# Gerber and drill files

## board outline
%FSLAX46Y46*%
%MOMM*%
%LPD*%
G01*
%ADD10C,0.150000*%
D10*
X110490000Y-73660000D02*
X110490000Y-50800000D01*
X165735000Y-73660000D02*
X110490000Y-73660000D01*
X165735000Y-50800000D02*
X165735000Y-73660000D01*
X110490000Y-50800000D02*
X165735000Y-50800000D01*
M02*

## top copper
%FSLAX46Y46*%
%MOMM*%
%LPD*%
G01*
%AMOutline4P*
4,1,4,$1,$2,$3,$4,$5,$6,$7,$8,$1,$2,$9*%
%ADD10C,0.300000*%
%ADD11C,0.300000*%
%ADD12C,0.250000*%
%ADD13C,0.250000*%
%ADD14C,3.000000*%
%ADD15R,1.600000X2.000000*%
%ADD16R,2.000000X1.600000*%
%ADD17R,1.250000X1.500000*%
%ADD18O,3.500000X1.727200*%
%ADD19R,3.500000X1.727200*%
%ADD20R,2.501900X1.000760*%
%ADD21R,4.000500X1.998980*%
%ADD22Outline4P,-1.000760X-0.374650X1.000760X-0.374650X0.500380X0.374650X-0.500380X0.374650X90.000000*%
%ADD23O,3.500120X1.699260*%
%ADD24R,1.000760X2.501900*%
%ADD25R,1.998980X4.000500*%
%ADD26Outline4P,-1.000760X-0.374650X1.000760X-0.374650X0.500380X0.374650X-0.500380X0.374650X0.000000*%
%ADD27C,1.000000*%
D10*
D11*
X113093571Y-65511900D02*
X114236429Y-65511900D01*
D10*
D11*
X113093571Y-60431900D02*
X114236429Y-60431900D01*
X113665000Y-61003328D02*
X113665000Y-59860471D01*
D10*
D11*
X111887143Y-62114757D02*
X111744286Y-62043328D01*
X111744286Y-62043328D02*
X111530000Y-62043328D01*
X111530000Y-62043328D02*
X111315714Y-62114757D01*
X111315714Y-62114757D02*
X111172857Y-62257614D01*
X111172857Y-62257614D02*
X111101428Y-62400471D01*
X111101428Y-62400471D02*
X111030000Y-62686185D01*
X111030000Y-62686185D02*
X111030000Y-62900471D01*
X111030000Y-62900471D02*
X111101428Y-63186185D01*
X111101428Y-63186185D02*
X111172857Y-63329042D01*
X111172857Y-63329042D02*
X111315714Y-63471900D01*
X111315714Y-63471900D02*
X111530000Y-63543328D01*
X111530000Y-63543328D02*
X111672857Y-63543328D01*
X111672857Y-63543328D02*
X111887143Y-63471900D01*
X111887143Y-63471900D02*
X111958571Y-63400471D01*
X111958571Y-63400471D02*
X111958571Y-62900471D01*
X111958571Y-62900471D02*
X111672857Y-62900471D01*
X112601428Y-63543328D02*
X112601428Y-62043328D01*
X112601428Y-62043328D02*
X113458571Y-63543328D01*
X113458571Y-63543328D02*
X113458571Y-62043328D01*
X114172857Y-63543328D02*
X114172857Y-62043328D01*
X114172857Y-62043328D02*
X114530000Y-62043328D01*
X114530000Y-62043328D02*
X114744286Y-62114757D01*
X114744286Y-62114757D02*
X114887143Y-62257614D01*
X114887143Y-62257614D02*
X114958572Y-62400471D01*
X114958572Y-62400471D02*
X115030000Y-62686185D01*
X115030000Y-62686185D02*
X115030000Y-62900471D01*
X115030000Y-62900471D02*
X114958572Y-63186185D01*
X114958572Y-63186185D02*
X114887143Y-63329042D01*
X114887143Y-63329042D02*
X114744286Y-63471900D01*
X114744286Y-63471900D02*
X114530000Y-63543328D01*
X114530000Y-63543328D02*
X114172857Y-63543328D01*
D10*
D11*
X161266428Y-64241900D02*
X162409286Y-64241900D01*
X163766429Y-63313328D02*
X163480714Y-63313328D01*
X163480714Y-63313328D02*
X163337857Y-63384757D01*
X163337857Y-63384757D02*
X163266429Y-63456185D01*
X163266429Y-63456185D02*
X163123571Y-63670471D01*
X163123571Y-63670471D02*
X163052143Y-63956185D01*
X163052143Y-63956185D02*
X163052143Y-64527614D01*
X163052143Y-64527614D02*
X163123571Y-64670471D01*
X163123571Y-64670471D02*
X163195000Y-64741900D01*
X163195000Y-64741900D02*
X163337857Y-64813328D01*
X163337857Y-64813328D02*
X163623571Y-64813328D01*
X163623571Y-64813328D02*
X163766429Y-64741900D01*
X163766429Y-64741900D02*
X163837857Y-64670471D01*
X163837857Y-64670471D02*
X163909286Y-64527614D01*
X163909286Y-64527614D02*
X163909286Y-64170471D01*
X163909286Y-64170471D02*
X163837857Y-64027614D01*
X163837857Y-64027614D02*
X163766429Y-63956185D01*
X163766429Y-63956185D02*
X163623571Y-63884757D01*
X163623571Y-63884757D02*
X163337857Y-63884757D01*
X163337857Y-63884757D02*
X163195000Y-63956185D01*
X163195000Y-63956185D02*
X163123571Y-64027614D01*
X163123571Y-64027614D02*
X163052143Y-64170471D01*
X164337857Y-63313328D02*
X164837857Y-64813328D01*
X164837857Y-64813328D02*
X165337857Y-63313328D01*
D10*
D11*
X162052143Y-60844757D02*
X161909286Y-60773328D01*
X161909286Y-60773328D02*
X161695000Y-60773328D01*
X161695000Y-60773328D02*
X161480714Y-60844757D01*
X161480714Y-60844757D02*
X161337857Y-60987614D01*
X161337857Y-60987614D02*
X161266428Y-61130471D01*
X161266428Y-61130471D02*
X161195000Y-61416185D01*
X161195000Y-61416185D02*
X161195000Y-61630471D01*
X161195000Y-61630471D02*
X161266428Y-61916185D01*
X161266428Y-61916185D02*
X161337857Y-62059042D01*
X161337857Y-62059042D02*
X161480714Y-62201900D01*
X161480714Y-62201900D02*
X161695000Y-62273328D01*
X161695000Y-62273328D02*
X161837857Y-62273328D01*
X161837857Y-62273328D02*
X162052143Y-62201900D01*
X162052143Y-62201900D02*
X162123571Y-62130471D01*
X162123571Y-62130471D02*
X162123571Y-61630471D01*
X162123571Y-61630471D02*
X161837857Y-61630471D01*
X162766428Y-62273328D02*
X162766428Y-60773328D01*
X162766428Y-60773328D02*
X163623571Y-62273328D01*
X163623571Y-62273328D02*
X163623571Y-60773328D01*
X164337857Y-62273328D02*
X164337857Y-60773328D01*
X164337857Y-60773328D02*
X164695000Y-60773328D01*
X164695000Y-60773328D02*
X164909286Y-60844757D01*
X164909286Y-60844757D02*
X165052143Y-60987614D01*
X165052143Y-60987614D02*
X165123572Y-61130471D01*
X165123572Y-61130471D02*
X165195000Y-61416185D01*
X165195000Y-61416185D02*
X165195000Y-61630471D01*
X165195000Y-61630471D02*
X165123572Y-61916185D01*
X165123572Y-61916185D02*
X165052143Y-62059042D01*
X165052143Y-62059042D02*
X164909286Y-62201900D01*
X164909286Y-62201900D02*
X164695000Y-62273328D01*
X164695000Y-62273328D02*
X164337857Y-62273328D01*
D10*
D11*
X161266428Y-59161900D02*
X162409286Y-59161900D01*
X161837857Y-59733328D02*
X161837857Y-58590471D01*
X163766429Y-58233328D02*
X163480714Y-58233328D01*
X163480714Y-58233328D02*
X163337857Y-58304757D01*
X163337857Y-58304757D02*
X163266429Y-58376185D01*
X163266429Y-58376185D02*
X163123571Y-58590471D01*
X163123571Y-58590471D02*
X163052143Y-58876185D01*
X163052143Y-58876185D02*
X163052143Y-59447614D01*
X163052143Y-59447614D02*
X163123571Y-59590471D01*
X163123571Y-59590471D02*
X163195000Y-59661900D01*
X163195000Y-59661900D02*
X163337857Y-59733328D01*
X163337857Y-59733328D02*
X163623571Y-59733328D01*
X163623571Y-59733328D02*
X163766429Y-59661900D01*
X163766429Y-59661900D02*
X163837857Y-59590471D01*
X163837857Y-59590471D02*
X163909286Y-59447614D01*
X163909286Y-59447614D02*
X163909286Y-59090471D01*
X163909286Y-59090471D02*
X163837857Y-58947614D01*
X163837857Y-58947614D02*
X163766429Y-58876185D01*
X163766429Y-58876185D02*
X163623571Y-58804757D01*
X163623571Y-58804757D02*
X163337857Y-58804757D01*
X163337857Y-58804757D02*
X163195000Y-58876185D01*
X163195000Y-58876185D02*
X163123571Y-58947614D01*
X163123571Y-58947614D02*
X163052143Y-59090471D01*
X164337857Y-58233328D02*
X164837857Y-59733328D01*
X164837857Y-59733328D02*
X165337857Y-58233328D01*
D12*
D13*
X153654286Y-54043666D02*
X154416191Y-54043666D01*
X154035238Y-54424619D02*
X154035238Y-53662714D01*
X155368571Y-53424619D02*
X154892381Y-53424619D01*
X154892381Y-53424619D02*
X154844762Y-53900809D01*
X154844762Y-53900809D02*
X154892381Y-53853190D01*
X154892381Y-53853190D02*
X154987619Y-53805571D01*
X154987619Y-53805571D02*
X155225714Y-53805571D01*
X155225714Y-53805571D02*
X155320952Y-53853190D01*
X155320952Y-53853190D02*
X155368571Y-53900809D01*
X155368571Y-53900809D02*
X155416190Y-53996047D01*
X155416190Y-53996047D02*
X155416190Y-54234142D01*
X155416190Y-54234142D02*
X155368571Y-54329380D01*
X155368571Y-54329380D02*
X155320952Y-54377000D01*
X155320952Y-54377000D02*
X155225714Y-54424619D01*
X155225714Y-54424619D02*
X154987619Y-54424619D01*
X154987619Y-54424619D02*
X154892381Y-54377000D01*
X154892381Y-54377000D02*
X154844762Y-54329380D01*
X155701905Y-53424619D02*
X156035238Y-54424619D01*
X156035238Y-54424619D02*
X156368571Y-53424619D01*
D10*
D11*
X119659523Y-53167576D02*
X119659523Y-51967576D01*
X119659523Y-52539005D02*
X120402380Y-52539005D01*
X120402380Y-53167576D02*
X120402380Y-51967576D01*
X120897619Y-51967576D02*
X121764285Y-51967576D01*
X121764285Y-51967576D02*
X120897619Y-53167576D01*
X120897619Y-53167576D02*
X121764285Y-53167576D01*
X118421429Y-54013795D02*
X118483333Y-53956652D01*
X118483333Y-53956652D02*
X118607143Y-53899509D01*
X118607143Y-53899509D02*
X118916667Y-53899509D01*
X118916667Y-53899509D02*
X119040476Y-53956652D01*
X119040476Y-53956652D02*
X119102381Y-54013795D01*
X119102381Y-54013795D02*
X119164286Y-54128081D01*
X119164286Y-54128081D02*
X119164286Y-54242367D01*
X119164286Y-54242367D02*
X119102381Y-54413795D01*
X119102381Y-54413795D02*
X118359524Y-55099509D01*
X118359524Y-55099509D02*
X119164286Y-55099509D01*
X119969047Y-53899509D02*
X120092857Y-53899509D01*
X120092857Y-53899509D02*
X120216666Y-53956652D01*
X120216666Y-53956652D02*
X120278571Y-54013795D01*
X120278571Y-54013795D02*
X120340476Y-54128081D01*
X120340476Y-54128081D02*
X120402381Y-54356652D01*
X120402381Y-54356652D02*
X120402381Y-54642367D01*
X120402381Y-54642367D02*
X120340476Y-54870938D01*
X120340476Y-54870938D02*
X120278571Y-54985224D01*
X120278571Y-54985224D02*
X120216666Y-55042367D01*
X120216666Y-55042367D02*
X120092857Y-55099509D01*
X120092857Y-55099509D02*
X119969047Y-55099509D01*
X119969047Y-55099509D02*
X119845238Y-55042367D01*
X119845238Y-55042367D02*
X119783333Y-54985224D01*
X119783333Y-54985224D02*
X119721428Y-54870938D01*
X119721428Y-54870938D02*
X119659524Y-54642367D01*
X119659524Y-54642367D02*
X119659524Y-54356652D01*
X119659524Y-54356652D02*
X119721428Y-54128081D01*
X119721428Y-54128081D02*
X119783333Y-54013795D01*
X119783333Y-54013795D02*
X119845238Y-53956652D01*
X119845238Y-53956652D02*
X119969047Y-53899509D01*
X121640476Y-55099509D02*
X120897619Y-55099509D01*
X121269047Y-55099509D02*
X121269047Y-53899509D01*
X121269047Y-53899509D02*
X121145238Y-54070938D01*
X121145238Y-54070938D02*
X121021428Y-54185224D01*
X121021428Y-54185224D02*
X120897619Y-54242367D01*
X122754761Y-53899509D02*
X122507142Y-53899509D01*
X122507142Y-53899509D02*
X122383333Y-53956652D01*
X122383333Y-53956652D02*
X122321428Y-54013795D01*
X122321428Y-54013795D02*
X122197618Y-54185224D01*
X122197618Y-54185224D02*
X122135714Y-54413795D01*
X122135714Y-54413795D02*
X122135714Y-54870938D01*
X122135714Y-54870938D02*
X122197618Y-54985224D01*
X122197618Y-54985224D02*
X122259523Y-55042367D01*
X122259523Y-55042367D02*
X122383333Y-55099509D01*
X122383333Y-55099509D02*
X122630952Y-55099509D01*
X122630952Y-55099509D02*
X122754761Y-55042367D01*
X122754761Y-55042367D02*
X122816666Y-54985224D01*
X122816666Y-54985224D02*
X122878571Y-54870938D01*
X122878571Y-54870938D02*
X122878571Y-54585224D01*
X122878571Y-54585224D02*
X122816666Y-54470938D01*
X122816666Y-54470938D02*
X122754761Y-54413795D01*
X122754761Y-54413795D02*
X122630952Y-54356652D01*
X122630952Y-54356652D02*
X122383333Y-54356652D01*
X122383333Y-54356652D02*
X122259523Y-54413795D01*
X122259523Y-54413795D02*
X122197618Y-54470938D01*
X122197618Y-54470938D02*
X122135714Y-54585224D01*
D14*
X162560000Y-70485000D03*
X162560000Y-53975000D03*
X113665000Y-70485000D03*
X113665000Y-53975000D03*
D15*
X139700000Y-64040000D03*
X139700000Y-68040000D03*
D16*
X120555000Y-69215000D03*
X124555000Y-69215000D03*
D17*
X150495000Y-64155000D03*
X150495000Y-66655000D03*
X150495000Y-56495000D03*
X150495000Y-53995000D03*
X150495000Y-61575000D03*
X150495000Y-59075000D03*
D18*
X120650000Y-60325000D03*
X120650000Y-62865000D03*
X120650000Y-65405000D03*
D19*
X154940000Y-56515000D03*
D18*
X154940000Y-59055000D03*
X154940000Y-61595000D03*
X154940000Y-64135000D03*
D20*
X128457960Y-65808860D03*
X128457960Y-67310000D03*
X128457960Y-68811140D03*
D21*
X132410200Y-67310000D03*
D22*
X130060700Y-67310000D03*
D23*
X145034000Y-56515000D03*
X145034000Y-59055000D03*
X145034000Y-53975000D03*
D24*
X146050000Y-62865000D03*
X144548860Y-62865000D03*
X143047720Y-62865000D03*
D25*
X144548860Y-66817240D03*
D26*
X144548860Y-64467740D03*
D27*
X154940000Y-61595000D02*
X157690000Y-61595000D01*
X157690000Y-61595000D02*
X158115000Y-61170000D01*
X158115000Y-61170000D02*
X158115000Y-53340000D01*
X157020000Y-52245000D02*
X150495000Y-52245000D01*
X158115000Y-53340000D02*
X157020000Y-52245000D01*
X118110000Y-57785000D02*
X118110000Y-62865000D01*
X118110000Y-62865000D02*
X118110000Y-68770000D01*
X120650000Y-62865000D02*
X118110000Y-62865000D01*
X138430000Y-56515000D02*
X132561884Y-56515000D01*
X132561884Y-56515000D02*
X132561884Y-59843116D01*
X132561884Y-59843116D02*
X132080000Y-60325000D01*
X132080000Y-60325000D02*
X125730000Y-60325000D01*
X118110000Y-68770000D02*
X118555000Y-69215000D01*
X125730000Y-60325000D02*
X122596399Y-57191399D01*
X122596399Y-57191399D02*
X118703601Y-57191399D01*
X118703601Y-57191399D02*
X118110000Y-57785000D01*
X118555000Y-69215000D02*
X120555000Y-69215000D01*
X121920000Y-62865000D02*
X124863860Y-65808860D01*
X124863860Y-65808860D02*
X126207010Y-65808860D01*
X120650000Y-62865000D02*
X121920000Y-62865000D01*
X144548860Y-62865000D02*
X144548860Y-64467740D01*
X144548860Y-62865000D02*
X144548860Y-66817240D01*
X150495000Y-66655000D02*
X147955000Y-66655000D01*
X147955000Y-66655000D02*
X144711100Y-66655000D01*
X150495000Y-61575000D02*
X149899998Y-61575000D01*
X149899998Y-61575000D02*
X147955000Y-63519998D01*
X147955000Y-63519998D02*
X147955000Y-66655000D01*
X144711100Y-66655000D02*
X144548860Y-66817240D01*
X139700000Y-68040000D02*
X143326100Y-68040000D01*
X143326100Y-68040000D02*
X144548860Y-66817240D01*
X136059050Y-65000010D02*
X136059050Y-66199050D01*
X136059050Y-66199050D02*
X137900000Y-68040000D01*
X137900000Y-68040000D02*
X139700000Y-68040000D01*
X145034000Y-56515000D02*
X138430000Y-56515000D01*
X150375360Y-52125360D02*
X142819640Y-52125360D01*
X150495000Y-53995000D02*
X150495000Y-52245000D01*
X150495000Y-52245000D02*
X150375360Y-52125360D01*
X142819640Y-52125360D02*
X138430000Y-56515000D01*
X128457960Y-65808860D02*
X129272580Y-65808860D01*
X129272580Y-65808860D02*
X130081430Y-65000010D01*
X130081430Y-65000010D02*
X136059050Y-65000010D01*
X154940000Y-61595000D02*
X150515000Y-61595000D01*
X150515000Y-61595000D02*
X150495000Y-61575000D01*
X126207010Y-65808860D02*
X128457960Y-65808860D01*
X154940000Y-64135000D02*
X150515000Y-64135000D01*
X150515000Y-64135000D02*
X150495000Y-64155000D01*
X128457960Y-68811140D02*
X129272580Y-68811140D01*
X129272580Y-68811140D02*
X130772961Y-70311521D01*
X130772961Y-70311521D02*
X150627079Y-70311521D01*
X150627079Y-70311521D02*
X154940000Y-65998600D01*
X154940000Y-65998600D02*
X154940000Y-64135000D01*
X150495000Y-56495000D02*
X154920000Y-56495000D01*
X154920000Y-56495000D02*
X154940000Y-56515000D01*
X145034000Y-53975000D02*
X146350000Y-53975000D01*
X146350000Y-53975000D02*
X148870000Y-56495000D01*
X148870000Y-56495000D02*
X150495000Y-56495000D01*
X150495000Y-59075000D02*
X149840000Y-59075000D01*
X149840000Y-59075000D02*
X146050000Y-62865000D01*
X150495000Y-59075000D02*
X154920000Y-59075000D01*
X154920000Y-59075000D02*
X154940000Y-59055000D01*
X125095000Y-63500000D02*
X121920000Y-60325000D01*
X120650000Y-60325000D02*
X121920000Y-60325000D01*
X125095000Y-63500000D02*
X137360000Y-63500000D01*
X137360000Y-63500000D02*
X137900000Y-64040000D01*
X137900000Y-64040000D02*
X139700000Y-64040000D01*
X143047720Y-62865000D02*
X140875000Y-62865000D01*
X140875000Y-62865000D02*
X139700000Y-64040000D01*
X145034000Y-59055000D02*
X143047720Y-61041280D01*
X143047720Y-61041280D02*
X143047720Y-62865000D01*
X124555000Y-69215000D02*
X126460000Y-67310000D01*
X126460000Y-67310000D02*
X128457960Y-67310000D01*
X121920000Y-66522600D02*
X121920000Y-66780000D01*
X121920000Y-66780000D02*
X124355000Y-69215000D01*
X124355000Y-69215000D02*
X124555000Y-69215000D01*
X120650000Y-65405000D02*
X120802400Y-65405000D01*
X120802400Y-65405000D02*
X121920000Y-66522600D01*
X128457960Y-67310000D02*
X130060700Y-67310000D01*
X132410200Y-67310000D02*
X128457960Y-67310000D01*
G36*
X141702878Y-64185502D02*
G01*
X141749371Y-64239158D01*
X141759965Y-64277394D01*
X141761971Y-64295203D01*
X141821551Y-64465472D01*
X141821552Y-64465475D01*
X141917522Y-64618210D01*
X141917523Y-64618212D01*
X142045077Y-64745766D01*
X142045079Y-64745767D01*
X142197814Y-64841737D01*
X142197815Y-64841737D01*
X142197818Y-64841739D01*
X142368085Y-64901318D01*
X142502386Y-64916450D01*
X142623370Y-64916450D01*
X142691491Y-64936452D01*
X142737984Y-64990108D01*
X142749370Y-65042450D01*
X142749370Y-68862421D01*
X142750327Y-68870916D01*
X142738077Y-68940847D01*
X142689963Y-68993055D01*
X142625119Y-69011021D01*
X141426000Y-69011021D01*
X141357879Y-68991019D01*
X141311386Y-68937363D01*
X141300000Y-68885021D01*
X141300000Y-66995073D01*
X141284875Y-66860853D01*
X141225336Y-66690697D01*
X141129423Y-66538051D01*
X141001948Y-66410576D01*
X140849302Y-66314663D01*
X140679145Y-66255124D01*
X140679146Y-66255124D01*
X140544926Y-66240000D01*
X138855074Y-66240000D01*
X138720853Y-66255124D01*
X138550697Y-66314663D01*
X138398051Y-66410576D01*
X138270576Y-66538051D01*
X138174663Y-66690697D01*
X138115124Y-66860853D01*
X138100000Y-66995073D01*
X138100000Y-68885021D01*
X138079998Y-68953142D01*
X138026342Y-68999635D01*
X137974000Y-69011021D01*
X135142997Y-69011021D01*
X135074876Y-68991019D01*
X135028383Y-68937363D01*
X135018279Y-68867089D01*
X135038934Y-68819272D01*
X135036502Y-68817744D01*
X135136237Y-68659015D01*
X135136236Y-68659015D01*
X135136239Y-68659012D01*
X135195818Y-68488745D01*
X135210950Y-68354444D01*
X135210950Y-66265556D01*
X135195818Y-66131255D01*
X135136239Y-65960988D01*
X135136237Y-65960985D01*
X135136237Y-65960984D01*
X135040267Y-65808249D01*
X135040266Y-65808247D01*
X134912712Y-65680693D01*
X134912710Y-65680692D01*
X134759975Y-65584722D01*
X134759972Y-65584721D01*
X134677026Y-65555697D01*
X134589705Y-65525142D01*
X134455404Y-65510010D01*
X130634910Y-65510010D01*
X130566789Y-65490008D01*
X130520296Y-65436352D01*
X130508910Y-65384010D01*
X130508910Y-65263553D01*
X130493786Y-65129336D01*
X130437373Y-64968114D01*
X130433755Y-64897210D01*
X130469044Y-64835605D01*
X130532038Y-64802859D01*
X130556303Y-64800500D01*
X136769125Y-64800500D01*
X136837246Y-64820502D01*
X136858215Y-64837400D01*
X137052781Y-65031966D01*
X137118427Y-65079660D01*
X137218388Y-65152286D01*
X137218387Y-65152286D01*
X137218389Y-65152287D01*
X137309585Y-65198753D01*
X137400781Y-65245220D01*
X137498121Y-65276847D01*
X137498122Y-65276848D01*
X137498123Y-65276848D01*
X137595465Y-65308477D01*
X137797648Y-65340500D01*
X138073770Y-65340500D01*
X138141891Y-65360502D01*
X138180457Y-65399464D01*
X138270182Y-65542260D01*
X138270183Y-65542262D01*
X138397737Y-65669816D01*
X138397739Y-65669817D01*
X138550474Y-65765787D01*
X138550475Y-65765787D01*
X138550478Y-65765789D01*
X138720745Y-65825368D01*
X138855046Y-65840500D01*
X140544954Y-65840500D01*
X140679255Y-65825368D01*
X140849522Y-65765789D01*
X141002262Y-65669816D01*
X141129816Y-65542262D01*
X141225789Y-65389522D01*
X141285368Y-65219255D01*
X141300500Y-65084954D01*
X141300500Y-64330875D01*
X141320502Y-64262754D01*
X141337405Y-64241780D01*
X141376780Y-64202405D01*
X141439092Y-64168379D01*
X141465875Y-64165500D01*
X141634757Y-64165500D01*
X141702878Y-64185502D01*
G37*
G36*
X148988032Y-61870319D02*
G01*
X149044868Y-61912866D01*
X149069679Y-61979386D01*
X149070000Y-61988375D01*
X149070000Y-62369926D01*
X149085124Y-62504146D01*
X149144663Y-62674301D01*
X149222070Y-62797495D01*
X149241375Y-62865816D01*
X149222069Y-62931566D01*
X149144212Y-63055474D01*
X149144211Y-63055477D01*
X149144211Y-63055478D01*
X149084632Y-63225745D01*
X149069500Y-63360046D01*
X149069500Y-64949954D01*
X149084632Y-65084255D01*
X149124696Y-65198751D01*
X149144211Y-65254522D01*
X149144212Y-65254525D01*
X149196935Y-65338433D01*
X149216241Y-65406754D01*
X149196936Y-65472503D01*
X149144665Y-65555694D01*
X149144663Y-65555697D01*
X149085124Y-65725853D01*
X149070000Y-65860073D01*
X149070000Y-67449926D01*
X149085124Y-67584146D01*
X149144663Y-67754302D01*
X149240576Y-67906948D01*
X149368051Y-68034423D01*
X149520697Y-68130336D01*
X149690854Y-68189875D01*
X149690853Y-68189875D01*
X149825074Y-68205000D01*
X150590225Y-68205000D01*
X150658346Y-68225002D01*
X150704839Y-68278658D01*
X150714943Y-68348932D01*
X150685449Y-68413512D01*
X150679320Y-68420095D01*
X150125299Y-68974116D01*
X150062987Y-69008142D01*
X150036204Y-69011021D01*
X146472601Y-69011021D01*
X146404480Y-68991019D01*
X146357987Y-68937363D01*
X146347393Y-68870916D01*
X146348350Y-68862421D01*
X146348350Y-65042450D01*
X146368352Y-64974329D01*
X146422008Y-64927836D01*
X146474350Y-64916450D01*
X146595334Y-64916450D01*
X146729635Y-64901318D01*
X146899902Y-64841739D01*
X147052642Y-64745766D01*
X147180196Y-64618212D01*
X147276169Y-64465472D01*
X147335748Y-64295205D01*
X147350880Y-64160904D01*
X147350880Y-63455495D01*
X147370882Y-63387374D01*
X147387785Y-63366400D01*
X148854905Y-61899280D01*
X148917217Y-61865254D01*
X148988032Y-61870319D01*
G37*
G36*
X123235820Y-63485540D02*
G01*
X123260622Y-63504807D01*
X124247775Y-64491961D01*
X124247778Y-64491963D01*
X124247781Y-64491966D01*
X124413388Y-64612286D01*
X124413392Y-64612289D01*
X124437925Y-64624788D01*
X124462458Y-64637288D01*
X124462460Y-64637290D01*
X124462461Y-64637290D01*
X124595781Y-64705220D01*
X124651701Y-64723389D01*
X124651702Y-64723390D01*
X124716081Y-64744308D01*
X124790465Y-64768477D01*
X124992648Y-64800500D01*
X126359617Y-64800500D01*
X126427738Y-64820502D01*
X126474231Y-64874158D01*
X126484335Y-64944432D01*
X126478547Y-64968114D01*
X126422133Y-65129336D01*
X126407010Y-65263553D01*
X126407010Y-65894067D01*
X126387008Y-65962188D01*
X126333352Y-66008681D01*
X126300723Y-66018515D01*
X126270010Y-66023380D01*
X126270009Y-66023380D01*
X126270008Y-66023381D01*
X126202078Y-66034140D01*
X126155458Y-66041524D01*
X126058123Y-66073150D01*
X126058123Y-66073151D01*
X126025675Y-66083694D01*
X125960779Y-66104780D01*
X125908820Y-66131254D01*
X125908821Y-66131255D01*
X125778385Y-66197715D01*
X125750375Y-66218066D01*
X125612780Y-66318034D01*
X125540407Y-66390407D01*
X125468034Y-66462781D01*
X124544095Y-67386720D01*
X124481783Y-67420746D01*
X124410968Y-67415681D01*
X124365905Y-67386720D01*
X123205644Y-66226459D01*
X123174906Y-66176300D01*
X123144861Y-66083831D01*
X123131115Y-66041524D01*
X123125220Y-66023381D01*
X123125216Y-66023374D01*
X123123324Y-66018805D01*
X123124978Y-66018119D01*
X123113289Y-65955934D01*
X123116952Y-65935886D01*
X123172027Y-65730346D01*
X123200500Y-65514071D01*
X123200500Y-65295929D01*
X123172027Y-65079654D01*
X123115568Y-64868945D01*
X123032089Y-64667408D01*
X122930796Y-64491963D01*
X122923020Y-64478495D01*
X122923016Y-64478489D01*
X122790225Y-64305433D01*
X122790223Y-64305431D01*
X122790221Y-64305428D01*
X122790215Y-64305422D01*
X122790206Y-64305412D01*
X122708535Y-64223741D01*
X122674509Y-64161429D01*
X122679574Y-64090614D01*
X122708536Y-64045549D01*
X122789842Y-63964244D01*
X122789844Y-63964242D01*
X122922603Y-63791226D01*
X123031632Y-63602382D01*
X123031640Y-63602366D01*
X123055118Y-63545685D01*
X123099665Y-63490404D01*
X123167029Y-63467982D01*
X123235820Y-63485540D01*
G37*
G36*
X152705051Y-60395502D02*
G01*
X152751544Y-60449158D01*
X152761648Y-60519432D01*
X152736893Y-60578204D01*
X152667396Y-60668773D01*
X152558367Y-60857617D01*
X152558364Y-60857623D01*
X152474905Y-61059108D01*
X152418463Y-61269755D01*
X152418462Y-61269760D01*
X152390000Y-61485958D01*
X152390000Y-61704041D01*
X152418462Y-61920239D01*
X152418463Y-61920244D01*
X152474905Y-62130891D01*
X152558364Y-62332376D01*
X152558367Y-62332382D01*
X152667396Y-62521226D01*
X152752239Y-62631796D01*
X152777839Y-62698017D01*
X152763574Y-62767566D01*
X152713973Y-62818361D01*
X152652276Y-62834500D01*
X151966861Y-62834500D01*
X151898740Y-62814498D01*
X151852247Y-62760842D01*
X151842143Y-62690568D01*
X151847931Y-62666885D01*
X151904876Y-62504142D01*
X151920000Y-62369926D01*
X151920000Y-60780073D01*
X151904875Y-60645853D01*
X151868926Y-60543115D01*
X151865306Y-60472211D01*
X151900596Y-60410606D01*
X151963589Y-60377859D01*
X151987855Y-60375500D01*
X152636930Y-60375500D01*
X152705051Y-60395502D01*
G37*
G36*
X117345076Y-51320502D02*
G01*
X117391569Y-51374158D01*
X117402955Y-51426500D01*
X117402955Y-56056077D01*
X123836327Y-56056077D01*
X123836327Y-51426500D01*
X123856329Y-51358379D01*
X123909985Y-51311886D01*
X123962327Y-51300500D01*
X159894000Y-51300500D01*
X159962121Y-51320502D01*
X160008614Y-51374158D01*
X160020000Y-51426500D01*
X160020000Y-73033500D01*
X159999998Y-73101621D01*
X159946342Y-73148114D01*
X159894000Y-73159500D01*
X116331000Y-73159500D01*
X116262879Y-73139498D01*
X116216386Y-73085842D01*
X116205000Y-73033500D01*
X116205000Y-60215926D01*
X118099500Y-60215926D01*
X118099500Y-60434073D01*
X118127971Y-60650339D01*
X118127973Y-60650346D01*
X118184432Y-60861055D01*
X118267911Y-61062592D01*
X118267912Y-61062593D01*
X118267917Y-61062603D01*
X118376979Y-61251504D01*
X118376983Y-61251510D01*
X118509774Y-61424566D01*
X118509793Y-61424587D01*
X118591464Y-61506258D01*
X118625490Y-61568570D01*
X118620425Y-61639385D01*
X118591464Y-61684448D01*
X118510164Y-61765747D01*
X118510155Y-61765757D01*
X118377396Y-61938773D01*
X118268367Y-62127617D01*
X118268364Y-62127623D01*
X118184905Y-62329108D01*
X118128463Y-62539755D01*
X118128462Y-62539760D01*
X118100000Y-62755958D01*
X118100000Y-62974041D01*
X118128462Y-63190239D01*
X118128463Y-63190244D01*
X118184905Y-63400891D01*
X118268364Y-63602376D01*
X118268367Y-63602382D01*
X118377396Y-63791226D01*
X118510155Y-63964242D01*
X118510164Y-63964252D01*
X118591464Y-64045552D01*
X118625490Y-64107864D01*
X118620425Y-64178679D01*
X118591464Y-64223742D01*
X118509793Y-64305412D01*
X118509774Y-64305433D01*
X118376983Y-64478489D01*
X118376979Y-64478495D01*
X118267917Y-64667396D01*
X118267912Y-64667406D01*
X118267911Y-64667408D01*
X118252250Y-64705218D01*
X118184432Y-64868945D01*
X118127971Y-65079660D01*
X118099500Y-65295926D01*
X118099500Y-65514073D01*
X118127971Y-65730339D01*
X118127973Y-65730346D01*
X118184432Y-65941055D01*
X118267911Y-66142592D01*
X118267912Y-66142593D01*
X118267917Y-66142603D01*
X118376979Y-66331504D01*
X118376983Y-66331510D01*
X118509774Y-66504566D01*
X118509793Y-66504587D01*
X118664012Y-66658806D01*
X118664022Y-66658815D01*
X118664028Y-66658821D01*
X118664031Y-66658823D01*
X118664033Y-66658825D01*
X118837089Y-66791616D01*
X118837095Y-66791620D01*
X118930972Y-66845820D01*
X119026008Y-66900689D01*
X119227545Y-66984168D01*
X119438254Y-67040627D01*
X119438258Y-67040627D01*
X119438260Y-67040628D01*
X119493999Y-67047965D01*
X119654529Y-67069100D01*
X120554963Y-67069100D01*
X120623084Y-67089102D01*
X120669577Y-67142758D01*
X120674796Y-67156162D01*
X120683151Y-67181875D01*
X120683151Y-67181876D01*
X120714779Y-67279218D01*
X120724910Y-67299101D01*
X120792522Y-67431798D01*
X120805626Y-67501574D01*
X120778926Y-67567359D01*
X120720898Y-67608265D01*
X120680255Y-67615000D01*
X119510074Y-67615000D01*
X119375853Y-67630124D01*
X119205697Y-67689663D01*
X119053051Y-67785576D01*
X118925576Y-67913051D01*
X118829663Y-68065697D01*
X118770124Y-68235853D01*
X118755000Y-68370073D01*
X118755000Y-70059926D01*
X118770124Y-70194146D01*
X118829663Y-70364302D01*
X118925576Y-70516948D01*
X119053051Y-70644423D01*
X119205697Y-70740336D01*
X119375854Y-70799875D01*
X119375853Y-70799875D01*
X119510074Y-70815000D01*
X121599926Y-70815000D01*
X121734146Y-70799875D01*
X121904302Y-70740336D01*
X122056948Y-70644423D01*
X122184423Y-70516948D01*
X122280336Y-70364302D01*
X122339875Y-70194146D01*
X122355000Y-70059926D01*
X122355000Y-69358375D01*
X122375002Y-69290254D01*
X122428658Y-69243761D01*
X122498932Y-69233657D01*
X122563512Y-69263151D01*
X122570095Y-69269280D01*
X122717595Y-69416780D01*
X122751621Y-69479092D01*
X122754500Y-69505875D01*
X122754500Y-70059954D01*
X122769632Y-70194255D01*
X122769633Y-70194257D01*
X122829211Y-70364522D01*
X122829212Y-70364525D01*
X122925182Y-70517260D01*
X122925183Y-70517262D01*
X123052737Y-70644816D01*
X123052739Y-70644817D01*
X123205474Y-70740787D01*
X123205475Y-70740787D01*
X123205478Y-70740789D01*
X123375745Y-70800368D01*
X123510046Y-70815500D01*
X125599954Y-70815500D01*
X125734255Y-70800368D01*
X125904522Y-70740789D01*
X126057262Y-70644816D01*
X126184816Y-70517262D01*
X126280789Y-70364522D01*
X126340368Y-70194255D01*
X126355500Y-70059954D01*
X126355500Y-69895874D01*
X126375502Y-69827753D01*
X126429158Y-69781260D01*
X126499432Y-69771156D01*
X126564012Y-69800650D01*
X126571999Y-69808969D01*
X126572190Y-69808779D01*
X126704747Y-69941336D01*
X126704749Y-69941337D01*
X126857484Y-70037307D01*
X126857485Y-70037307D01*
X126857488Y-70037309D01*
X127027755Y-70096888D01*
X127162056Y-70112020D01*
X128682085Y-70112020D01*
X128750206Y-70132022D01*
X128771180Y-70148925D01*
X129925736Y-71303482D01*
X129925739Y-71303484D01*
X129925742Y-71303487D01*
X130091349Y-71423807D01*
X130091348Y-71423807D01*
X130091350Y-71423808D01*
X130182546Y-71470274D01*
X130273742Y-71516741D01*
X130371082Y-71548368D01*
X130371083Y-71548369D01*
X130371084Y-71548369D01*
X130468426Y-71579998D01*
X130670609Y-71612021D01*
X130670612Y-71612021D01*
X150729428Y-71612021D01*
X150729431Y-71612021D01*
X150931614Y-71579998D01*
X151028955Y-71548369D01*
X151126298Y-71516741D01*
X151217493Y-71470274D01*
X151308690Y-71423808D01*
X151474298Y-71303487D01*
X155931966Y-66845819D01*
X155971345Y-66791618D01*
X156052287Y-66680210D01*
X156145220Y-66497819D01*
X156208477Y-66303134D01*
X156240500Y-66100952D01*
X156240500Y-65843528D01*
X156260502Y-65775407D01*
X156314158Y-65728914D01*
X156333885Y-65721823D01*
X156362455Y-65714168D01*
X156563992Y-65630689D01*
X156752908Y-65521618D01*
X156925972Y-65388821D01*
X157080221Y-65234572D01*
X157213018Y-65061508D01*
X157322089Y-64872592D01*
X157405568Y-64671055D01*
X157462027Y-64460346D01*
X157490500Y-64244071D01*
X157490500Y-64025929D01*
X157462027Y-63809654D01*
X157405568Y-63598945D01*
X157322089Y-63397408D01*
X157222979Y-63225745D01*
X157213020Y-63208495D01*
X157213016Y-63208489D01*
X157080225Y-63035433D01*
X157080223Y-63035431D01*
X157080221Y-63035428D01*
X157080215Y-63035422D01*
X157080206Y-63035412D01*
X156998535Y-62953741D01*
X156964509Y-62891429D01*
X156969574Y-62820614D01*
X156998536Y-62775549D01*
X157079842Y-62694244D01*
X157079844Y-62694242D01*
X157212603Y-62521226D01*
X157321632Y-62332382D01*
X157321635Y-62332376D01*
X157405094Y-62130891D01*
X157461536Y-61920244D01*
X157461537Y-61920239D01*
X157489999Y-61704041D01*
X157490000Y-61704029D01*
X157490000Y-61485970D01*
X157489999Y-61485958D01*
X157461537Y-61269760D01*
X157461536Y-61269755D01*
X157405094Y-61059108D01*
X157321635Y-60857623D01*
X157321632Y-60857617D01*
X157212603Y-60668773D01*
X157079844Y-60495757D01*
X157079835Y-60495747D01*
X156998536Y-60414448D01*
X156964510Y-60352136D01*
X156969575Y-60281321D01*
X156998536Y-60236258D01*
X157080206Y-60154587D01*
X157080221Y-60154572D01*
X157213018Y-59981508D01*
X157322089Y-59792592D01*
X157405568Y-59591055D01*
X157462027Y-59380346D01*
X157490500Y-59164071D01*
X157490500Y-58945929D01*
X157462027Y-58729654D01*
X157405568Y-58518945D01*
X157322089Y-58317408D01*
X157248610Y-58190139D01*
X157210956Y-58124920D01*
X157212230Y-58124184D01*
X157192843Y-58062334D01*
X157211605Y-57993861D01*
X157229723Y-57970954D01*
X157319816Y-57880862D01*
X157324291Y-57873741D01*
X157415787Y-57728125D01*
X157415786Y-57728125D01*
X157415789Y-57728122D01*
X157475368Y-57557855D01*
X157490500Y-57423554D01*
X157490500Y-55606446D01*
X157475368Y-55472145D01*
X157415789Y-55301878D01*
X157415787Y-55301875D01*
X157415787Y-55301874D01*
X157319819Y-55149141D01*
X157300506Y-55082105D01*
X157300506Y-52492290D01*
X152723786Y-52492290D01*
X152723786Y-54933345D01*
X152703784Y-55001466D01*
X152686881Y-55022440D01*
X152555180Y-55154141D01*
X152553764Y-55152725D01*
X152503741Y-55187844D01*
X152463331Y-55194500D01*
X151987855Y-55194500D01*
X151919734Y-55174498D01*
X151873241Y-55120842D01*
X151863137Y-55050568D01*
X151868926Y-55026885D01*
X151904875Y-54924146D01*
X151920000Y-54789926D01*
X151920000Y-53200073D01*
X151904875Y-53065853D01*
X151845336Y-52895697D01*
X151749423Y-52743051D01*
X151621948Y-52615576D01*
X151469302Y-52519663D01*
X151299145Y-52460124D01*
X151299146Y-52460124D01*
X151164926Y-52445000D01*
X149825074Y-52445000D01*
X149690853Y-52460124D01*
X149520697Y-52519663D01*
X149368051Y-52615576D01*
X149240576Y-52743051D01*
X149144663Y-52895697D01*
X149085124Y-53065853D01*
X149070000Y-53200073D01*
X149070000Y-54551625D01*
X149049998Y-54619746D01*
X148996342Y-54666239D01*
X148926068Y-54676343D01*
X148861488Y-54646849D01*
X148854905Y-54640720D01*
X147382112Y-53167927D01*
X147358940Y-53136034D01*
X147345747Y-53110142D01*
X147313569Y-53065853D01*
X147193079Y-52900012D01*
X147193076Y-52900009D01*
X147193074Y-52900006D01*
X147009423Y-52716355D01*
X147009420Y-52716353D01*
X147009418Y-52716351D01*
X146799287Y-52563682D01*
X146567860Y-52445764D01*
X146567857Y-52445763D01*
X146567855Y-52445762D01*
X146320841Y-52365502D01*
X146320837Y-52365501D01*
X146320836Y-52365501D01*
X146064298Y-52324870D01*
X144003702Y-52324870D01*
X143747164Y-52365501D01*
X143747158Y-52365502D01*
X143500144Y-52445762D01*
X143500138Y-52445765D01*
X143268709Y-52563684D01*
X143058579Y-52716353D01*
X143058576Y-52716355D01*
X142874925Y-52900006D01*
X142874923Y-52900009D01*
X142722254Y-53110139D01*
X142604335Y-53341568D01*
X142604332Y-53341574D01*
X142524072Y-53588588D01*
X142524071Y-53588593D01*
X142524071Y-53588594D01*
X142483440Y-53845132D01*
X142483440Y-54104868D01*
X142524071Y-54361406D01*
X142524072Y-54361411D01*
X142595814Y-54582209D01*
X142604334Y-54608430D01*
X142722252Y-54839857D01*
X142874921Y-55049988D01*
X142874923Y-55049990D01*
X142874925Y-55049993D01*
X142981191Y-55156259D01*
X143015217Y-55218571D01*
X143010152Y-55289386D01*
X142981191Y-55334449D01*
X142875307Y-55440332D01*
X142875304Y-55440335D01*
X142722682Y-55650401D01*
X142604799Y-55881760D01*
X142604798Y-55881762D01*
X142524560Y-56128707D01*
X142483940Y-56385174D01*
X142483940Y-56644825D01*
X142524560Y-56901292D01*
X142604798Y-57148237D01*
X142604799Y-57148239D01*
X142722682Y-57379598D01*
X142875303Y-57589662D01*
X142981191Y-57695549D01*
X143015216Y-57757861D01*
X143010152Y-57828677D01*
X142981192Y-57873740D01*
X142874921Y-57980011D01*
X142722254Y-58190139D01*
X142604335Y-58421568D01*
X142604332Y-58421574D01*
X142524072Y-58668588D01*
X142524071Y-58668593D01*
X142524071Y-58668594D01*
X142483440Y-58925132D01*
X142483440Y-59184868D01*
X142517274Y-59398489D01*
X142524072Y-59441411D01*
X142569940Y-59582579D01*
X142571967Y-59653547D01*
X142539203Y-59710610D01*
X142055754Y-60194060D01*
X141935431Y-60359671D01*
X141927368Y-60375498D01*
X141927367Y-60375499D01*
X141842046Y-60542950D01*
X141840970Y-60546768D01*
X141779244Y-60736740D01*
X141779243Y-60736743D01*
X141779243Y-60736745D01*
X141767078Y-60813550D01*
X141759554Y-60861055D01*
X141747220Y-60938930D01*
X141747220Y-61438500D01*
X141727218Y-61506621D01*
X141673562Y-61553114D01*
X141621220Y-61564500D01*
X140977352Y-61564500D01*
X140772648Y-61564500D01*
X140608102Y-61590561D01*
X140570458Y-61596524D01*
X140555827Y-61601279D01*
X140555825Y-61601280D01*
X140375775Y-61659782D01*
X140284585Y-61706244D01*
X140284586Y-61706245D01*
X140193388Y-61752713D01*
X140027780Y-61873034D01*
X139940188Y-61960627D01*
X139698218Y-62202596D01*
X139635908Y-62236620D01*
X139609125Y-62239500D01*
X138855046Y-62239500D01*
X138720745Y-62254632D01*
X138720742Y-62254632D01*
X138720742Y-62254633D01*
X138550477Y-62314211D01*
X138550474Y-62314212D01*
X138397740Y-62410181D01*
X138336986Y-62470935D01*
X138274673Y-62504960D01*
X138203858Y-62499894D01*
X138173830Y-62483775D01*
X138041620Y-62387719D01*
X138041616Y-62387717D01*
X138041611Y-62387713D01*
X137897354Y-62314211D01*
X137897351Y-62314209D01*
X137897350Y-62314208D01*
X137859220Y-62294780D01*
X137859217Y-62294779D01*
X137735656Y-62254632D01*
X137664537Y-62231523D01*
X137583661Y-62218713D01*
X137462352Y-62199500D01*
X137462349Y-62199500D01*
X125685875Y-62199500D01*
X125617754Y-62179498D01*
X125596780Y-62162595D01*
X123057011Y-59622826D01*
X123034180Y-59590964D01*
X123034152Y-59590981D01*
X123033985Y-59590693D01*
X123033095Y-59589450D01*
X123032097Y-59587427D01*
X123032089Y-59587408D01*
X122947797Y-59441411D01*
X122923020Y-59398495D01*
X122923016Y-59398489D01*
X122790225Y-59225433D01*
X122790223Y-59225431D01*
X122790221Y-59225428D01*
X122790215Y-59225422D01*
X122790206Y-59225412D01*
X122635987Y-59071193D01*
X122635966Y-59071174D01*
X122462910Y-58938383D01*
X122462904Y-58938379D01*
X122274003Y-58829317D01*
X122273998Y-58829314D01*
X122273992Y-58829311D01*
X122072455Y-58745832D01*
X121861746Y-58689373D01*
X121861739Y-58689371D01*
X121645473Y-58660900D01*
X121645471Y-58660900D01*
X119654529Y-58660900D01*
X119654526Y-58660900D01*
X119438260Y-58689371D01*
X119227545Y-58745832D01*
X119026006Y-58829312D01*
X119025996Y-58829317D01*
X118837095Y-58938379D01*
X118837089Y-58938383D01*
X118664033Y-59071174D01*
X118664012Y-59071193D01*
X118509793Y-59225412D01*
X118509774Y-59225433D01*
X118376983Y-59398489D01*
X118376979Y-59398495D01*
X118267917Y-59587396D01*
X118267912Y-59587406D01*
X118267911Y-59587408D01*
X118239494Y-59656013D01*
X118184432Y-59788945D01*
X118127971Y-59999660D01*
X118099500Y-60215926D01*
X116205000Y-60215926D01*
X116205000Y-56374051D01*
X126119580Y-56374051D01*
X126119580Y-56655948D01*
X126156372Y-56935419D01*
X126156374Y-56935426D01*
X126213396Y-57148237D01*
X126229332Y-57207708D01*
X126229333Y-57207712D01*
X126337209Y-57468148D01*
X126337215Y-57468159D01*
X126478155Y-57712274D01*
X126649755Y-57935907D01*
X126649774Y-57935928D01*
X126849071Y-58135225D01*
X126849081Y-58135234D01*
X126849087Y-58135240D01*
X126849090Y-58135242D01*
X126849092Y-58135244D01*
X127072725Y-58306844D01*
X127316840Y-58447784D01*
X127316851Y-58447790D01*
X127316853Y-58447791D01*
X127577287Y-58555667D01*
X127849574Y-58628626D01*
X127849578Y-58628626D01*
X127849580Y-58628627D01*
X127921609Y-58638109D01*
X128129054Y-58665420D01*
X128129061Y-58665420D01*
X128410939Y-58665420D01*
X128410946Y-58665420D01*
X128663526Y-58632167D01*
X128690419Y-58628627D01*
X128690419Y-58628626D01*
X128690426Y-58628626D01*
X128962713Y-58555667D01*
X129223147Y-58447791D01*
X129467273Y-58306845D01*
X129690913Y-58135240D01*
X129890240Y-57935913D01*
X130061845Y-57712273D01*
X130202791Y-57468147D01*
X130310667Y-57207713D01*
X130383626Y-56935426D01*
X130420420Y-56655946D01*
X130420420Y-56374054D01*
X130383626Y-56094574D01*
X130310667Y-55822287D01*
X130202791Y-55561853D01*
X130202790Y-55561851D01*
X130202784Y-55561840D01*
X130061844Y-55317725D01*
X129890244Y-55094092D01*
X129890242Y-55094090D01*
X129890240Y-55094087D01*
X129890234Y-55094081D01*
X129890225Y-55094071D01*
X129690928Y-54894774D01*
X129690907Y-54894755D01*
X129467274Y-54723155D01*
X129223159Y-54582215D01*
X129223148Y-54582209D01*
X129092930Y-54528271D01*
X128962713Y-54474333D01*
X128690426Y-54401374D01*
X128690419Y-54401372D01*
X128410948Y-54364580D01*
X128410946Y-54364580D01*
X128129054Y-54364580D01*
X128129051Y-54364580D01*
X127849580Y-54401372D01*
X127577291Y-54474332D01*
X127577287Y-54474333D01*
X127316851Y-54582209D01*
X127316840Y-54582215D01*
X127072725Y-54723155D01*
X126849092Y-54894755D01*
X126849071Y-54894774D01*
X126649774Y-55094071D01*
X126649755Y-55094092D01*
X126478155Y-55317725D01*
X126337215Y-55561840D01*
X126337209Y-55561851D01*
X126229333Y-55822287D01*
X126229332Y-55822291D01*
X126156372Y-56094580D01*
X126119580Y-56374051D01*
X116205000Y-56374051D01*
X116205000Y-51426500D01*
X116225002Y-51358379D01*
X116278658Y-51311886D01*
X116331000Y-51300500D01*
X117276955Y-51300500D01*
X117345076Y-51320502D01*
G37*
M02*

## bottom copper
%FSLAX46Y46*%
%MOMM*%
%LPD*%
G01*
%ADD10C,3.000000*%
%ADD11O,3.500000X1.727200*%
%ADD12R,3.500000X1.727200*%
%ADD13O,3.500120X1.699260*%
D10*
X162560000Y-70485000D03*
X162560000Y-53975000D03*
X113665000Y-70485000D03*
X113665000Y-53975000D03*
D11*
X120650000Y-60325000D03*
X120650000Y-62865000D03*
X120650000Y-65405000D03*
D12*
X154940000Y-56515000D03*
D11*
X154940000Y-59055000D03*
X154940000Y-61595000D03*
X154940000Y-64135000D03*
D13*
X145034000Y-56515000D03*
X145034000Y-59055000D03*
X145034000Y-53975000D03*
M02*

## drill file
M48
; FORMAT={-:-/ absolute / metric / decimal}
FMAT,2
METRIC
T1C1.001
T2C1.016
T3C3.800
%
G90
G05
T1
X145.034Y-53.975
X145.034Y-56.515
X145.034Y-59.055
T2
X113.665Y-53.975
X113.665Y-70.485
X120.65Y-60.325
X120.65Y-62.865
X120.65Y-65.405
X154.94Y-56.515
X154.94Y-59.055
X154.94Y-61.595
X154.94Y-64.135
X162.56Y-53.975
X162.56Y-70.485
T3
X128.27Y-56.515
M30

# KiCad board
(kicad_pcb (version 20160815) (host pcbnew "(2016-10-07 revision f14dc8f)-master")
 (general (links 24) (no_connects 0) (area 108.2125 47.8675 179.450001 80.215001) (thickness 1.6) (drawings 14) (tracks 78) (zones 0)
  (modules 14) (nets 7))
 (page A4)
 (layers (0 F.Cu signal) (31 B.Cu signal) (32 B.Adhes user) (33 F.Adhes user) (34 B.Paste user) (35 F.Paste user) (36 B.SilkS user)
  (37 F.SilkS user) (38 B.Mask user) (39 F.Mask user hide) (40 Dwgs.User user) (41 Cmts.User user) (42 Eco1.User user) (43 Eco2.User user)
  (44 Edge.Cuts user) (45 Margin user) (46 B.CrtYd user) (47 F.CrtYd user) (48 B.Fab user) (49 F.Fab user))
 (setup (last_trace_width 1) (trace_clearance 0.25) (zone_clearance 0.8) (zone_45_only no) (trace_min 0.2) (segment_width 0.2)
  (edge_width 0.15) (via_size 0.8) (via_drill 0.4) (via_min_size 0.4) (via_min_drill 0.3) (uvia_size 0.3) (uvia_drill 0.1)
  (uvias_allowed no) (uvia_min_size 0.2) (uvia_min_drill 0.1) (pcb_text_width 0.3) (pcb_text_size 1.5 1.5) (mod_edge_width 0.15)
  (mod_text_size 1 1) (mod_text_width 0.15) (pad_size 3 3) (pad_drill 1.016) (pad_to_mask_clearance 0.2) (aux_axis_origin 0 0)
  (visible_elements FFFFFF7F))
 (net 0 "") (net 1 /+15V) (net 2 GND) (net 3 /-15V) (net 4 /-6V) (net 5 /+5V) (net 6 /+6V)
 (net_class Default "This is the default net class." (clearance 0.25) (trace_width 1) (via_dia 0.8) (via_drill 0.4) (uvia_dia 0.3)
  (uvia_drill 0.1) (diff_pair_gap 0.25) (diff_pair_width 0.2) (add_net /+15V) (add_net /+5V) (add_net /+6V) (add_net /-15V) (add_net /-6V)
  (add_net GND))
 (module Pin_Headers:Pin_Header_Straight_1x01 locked (layer F.Cu) (at 162.56 70.485)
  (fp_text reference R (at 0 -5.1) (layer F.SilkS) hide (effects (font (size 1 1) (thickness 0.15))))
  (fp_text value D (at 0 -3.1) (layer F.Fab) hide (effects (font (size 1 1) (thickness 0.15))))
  (pad 1 thru_hole circle (at 0 0) (size 3 3) (drill 1.016) (layers *.Cu *.Mask F.SilkS)))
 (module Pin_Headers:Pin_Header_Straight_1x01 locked (layer F.Cu) (at 162.56 53.975)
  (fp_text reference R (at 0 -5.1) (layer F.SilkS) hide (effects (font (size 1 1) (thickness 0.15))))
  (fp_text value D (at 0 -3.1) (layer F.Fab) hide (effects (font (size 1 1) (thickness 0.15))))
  (pad 1 thru_hole circle (at 0 0) (size 3 3) (drill 1.016) (layers *.Cu *.Mask F.SilkS)))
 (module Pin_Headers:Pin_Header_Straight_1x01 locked (layer F.Cu) (at 113.665 70.485)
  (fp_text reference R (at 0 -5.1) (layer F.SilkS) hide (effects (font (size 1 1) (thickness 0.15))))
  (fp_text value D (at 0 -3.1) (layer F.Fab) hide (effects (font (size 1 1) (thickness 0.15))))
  (pad 1 thru_hole circle (at 0 0) (size 3 3) (drill 1.016) (layers *.Cu *.Mask F.SilkS)))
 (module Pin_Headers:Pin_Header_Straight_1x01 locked (layer F.Cu) (at 113.665 53.975)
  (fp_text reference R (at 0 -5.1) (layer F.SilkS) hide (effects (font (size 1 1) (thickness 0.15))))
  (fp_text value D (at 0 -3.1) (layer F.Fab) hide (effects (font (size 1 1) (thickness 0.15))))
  (pad 1 thru_hole circle (at 0 0) (size 3 3) (drill 1.016) (layers *.Cu *.Mask F.SilkS)))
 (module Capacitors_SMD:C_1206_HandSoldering (layer F.Cu) (at 139.7 66.04 270)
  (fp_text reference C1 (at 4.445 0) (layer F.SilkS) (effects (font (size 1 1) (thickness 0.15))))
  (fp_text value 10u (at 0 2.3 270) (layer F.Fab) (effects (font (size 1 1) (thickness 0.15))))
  (pad 1 smd rect (at -2 0 270) (size 2 1.6) (layers F.Cu F.Paste F.Mask) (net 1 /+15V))
  (pad 2 smd rect (at 2 0 270) (size 2 1.6) (layers F.Cu F.Paste F.Mask) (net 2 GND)))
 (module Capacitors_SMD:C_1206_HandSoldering (layer F.Cu) (at 122.555 69.215 180)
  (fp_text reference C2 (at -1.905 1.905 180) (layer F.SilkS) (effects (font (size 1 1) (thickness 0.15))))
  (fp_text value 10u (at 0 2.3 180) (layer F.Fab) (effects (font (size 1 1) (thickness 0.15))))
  (pad 2 smd rect (at 2 0 180) (size 2 1.6) (layers F.Cu F.Paste F.Mask) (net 2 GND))
  (pad 1 smd rect (at -2 0 180) (size 2 1.6) (layers F.Cu F.Paste F.Mask) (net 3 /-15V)))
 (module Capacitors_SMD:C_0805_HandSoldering (layer F.Cu) (at 150.495 65.405 270)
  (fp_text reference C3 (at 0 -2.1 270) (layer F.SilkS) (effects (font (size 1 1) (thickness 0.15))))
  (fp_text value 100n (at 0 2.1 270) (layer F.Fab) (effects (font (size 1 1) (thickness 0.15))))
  (pad 1 smd rect (at -1.25 0 270) (size 1.5 1.25) (layers F.Cu F.Paste F.Mask) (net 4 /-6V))
  (pad 2 smd rect (at 1.25 0 270) (size 1.5 1.25) (layers F.Cu F.Paste F.Mask) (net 2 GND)))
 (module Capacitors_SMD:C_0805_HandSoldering (layer F.Cu) (at 150.495 55.245 90)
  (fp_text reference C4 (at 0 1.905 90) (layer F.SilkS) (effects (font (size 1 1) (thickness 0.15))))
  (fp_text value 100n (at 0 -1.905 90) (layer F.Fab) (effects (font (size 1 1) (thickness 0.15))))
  (pad 1 smd rect (at -1.25 0 90) (size 1.5 1.25) (layers F.Cu F.Paste F.Mask) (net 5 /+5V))
  (pad 2 smd rect (at 1.25 0 90) (size 1.5 1.25) (layers F.Cu F.Paste F.Mask) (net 2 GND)))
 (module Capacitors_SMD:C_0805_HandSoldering (layer F.Cu) (at 150.495 60.325 270)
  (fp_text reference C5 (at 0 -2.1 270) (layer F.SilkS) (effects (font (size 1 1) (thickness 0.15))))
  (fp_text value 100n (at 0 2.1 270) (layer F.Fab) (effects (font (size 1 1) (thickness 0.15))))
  (pad 2 smd rect (at 1.25 0 270) (size 1.5 1.25) (layers F.Cu F.Paste F.Mask) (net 2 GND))
  (pad 1 smd rect (at -1.25 0 270) (size 1.5 1.25) (layers F.Cu F.Paste F.Mask) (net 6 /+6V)))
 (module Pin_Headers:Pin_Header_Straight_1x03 (layer F.Cu) (at 120.65 60.325)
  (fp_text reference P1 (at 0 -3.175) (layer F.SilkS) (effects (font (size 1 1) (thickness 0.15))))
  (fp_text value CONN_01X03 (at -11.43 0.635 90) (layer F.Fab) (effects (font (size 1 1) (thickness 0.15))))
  (pad 1 thru_hole oval (at 0 0) (size 3.5 1.7272) (drill 1.016) (layers *.Cu *.Mask F.SilkS) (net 1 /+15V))
  (pad 2 thru_hole oval (at 0 2.54) (size 3.5 1.7272) (drill 1.016) (layers *.Cu *.Mask F.SilkS) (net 2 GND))
  (pad 3 thru_hole oval (at 0 5.08) (size 3.5 1.7272) (drill 1.016) (layers *.Cu *.Mask F.SilkS) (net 3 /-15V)))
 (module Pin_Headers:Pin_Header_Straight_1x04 (layer F.Cu) (at 154.94 56.515)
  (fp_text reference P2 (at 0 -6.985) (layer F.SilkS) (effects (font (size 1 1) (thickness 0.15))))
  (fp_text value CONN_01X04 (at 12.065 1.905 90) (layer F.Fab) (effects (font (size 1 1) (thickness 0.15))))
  (pad 1 thru_hole rect (at 0 0) (size 3.5 1.7272) (drill 1.016) (layers *.Cu *.Mask F.SilkS) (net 5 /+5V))
  (pad 2 thru_hole oval (at 0 2.54) (size 3.5 1.7272) (drill 1.016) (layers *.Cu *.Mask F.SilkS) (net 6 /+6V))
  (pad 3 thru_hole oval (at 0 5.08) (size 3.5 1.7272) (drill 1.016) (layers *.Cu *.Mask F.SilkS) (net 2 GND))
  (pad 4 thru_hole oval (at 0 7.62) (size 3.5 1.7272) (drill 1.016) (layers *.Cu *.Mask F.SilkS) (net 4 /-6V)))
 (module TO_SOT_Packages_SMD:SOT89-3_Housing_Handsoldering (layer F.Cu) (at 130.81 67.31 270)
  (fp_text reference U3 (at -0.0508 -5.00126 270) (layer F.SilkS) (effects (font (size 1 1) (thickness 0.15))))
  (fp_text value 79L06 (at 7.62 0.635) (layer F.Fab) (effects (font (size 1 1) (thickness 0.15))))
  (pad 1 smd rect (at -1.50114 2.35204 270) (size 1.00076 2.5019) (layers F.Cu F.Paste F.Mask) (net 2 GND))
  (pad 2 smd rect (at 0 2.35204 270) (size 1.00076 2.5019) (layers F.Cu F.Paste F.Mask) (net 3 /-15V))
  (pad 3 smd rect (at 1.50114 2.35204 270) (size 1.00076 2.5019) (layers F.Cu F.Paste F.Mask) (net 4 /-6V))
  (pad 2 smd rect (at 0 -1.6002 270) (size 1.99898 4.0005) (layers F.Cu F.Paste F.Mask) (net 3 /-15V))
  (pad 2 smd trapezoid (at 0 0.7493 90) (size 1.50114 0.7493) (rect_delta 0 0.50038) (layers F.Cu F.Paste F.Mask) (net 3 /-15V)))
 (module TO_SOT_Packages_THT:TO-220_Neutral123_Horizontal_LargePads (layer F.Cu) (at 145.034 56.515 90)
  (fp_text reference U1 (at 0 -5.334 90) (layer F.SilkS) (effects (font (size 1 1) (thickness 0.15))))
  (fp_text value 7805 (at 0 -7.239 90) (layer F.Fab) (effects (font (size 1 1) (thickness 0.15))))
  (pad 2 thru_hole oval (at 0 0 180) (size 3.50012 1.69926) (drill 1.00076) (layers *.Cu *.Mask F.SilkS) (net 2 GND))
  (pad 1 thru_hole oval (at -2.54 0 180) (size 3.50012 1.69926) (drill 1.00076) (layers *.Cu *.Mask F.SilkS) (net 1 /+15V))
  (pad 3 thru_hole oval (at 2.54 0 180) (size 3.50012 1.69926) (drill 1.00076) (layers *.Cu *.Mask F.SilkS) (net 5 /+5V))
  (pad "" np_thru_hole circle (at 0 -16.764 180) (size 3.79984 3.79984) (drill 3.79984) (layers *.Cu *.Mask F.SilkS)))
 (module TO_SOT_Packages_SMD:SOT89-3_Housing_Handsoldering (layer F.Cu) (at 144.54886 65.21704 180)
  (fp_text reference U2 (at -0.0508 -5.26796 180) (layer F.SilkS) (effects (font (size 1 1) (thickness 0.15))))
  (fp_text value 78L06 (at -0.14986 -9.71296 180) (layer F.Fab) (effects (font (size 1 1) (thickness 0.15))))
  (pad 1 smd rect (at -1.50114 2.35204 180) (size 1.00076 2.5019) (layers F.Cu F.Paste F.Mask) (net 6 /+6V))
  (pad 2 smd rect (at 0 2.35204 180) (size 1.00076 2.5019) (layers F.Cu F.Paste F.Mask) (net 2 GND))
  (pad 3 smd rect (at 1.50114 2.35204 180) (size 1.00076 2.5019) (layers F.Cu F.Paste F.Mask) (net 1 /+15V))
  (pad 2 smd rect (at 0 -1.6002 180) (size 1.99898 4.0005) (layers F.Cu F.Paste F.Mask) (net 2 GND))
  (pad 2 smd trapezoid (at 0 0.7493) (size 1.50114 0.7493) (rect_delta 0 0.50038) (layers F.Cu F.Paste F.Mask) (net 2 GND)))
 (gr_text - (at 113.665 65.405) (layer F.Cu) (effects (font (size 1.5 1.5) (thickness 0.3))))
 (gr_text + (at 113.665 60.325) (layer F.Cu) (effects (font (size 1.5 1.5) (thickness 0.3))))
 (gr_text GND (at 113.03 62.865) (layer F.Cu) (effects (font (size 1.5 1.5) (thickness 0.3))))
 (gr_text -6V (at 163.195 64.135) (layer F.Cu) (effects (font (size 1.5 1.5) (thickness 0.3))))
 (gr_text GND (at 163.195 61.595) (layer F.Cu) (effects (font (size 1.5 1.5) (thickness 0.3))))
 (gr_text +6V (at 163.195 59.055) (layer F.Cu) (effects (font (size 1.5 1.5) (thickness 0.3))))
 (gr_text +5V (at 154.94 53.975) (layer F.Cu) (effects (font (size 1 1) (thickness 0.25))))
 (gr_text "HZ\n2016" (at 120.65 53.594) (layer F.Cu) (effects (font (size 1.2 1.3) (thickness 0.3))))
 (gr_line (start 110.49 73.66) (end 110.49 50.8) (layer Edge.Cuts) (width 0.15))
 (gr_line (start 165.735 73.66) (end 110.49 73.66) (layer Edge.Cuts) (width 0.15))
 (gr_line (start 165.735 50.8) (end 165.735 73.66) (layer Edge.Cuts) (width 0.15))
 (gr_line (start 110.49 50.8) (end 165.735 50.8) (layer Edge.Cuts) (width 0.15))
 (segment (start 154.94 61.595) (end 157.69 61.595) (width 1) (layer F.Cu) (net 2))
 (segment (start 157.69 61.595) (end 158.115 61.17) (width 1) (layer F.Cu) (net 2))
 (segment (start 158.115 61.17) (end 158.115 53.34) (width 1) (layer F.Cu) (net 2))
 (segment (start 157.02 52.245) (end 150.495 52.245) (width 1) (layer F.Cu) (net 2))
 (segment (start 158.115 53.34) (end 157.02 52.245) (width 1) (layer F.Cu) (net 2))
 (segment (start 118.11 57.785) (end 118.11 62.865) (width 1) (layer F.Cu) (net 2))
 (segment (start 118.11 62.865) (end 118.11 68.77) (width 1) (layer F.Cu) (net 2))
 (segment (start 120.65 62.865) (end 118.11 62.865) (width 1) (layer F.Cu) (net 2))
 (segment (start 138.43 56.515) (end 132.561884 56.515) (width 1) (layer F.Cu) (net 2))
 (segment (start 132.561884 56.515) (end 132.561884 59.843116) (width 1) (layer F.Cu) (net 2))
 (segment (start 132.561884 59.843116) (end 132.08 60.325) (width 1) (layer F.Cu) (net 2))
 (segment (start 132.08 60.325) (end 125.73 60.325) (width 1) (layer F.Cu) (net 2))
 (segment (start 118.11 68.77) (end 118.555 69.215) (width 1) (layer F.Cu) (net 2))
 (segment (start 125.73 60.325) (end 122.596399 57.191399) (width 1) (layer F.Cu) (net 2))
 (segment (start 122.596399 57.191399) (end 118.703601 57.191399) (width 1) (layer F.Cu) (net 2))
 (segment (start 118.703601 57.191399) (end 118.11 57.785) (width 1) (layer F.Cu) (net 2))
 (segment (start 118.555 69.215) (end 120.555 69.215) (width 1) (layer F.Cu) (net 2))
 (segment (start 121.92 62.865) (end 124.86386 65.80886) (width 1) (layer F.Cu) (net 2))
 (segment (start 124.86386 65.80886) (end 126.20701 65.80886) (width 1) (layer F.Cu) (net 2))
 (segment (start 120.65 62.865) (end 121.92 62.865) (width 1) (layer F.Cu) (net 2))
 (segment (start 144.54886 62.865) (end 144.54886 64.46774) (width 1) (layer F.Cu) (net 2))
 (segment (start 144.54886 62.865) (end 144.54886 66.81724) (width 1) (layer F.Cu) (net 2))
 (segment (start 150.495 66.655) (end 147.955 66.655) (width 1) (layer F.Cu) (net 2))
 (segment (start 147.955 66.655) (end 144.7111 66.655) (width 1) (layer F.Cu) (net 2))
 (segment (start 150.495 61.575) (end 149.899998 61.575) (width 1) (layer F.Cu) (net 2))
 (segment (start 149.899998 61.575) (end 147.955 63.519998) (width 1) (layer F.Cu) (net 2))
 (segment (start 147.955 63.519998) (end 147.955 66.655) (width 1) (layer F.Cu) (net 2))
 (segment (start 144.7111 66.655) (end 144.54886 66.81724) (width 1) (layer F.Cu) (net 2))
 (segment (start 139.7 68.04) (end 143.3261 68.04) (width 1) (layer F.Cu) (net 2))
 (segment (start 143.3261 68.04) (end 144.54886 66.81724) (width 1) (layer F.Cu) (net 2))
 (segment (start 136.05905 65.00001) (end 136.05905 66.19905) (width 1) (layer F.Cu) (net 2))
 (segment (start 136.05905 66.19905) (end 137.9 68.04) (width 1) (layer F.Cu) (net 2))
 (segment (start 137.9 68.04) (end 139.7 68.04) (width 1) (layer F.Cu) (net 2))
 (segment (start 145.034 56.515) (end 138.43 56.515) (width 1) (layer F.Cu) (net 2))
 (segment (start 150.37536 52.12536) (end 142.81964 52.12536) (width 1) (layer F.Cu) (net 2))
 (segment (start 150.495 53.995) (end 150.495 52.245) (width 1) (layer F.Cu) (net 2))
 (segment (start 150.495 52.245) (end 150.37536 52.12536) (width 1) (layer F.Cu) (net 2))
 (segment (start 142.81964 52.12536) (end 138.43 56.515) (width 1) (layer F.Cu) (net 2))
 (segment (start 128.45796 65.80886) (end 129.27258 65.80886) (width 1) (layer F.Cu) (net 2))
 (segment (start 129.27258 65.80886) (end 130.08143 65.00001) (width 1) (layer F.Cu) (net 2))
 (segment (start 130.08143 65.00001) (end 136.05905 65.00001) (width 1) (layer F.Cu) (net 2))
 (segment (start 154.94 61.595) (end 150.515 61.595) (width 1) (layer F.Cu) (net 2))
 (segment (start 150.515 61.595) (end 150.495 61.575) (width 1) (layer F.Cu) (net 2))
 (segment (start 126.20701 65.80886) (end 128.45796 65.80886) (width 1) (layer F.Cu) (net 2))
 (segment (start 154.94 64.135) (end 150.515 64.135) (width 1) (layer F.Cu) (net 4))
 (segment (start 150.515 64.135) (end 150.495 64.155) (width 1) (layer F.Cu) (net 4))
 (segment (start 128.45796 68.81114) (end 129.27258 68.81114) (width 1) (layer F.Cu) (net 4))
 (segment (start 129.27258 68.81114) (end 130.772961 70.311521) (width 1) (layer F.Cu) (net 4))
 (segment (start 130.772961 70.311521) (end 150.627079 70.311521) (width 1) (layer F.Cu) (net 4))
 (segment (start 150.627079 70.311521) (end 154.94 65.9986) (width 1) (layer F.Cu) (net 4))
 (segment (start 154.94 65.9986) (end 154.94 64.135) (width 1) (layer F.Cu) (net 4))
 (segment (start 150.495 56.495) (end 154.92 56.495) (width 1) (layer F.Cu) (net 5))
 (segment (start 154.92 56.495) (end 154.94 56.515) (width 1) (layer F.Cu) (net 5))
 (segment (start 145.034 53.975) (end 146.35 53.975) (width 1) (layer F.Cu) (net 5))
 (segment (start 146.35 53.975) (end 148.87 56.495) (width 1) (layer F.Cu) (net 5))
 (segment (start 148.87 56.495) (end 150.495 56.495) (width 1) (layer F.Cu) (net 5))
 (segment (start 150.495 59.075) (end 149.84 59.075) (width 1) (layer F.Cu) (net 6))
 (segment (start 149.84 59.075) (end 146.05 62.865) (width 1) (layer F.Cu) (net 6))
 (segment (start 150.495 59.075) (end 154.92 59.075) (width 1) (layer F.Cu) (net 6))
 (segment (start 154.92 59.075) (end 154.94 59.055) (width 1) (layer F.Cu) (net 6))
 (segment (start 125.095 63.5) (end 121.92 60.325) (width 1) (layer F.Cu) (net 1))
 (segment (start 120.65 60.325) (end 121.92 60.325) (width 1) (layer F.Cu) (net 1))
 (segment (start 125.095 63.5) (end 137.36 63.5) (width 1) (layer F.Cu) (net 1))
 (segment (start 137.36 63.5) (end 137.9 64.04) (width 1) (layer F.Cu) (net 1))
 (segment (start 137.9 64.04) (end 139.7 64.04) (width 1) (layer F.Cu) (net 1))
 (segment (start 143.04772 62.865) (end 140.875 62.865) (width 1) (layer F.Cu) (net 1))
 (segment (start 140.875 62.865) (end 139.7 64.04) (width 1) (layer F.Cu) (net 1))
 (segment (start 145.034 59.055) (end 143.04772 61.04128) (width 1) (layer F.Cu) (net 1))
 (segment (start 143.04772 61.04128) (end 143.04772 62.865) (width 1) (layer F.Cu) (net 1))
 (segment (start 124.555 69.215) (end 126.46 67.31) (width 1) (layer F.Cu) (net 3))
 (segment (start 126.46 67.31) (end 128.45796 67.31) (width 1) (layer F.Cu) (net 3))
 (segment (start 121.92 66.5226) (end 121.92 66.78) (width 1) (layer F.Cu) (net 3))
 (segment (start 121.92 66.78) (end 124.355 69.215) (width 1) (layer F.Cu) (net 3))
 (segment (start 124.355 69.215) (end 124.555 69.215) (width 1) (layer F.Cu) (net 3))
 (segment (start 120.65 65.405) (end 120.8024 65.405) (width 1) (layer F.Cu) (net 3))
 (segment (start 120.8024 65.405) (end 121.92 66.5226) (width 1) (layer F.Cu) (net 3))
 (segment (start 128.45796 67.31) (end 130.0607 67.31) (width 1) (layer F.Cu) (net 3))
 (segment (start 132.4102 67.31) (end 128.45796 67.31) (width 1) (layer F.Cu) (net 3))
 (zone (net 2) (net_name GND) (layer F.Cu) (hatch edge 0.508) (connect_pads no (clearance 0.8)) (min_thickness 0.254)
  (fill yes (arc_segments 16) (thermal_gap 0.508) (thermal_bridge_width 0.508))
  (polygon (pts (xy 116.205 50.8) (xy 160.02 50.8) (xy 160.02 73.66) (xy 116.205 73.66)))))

